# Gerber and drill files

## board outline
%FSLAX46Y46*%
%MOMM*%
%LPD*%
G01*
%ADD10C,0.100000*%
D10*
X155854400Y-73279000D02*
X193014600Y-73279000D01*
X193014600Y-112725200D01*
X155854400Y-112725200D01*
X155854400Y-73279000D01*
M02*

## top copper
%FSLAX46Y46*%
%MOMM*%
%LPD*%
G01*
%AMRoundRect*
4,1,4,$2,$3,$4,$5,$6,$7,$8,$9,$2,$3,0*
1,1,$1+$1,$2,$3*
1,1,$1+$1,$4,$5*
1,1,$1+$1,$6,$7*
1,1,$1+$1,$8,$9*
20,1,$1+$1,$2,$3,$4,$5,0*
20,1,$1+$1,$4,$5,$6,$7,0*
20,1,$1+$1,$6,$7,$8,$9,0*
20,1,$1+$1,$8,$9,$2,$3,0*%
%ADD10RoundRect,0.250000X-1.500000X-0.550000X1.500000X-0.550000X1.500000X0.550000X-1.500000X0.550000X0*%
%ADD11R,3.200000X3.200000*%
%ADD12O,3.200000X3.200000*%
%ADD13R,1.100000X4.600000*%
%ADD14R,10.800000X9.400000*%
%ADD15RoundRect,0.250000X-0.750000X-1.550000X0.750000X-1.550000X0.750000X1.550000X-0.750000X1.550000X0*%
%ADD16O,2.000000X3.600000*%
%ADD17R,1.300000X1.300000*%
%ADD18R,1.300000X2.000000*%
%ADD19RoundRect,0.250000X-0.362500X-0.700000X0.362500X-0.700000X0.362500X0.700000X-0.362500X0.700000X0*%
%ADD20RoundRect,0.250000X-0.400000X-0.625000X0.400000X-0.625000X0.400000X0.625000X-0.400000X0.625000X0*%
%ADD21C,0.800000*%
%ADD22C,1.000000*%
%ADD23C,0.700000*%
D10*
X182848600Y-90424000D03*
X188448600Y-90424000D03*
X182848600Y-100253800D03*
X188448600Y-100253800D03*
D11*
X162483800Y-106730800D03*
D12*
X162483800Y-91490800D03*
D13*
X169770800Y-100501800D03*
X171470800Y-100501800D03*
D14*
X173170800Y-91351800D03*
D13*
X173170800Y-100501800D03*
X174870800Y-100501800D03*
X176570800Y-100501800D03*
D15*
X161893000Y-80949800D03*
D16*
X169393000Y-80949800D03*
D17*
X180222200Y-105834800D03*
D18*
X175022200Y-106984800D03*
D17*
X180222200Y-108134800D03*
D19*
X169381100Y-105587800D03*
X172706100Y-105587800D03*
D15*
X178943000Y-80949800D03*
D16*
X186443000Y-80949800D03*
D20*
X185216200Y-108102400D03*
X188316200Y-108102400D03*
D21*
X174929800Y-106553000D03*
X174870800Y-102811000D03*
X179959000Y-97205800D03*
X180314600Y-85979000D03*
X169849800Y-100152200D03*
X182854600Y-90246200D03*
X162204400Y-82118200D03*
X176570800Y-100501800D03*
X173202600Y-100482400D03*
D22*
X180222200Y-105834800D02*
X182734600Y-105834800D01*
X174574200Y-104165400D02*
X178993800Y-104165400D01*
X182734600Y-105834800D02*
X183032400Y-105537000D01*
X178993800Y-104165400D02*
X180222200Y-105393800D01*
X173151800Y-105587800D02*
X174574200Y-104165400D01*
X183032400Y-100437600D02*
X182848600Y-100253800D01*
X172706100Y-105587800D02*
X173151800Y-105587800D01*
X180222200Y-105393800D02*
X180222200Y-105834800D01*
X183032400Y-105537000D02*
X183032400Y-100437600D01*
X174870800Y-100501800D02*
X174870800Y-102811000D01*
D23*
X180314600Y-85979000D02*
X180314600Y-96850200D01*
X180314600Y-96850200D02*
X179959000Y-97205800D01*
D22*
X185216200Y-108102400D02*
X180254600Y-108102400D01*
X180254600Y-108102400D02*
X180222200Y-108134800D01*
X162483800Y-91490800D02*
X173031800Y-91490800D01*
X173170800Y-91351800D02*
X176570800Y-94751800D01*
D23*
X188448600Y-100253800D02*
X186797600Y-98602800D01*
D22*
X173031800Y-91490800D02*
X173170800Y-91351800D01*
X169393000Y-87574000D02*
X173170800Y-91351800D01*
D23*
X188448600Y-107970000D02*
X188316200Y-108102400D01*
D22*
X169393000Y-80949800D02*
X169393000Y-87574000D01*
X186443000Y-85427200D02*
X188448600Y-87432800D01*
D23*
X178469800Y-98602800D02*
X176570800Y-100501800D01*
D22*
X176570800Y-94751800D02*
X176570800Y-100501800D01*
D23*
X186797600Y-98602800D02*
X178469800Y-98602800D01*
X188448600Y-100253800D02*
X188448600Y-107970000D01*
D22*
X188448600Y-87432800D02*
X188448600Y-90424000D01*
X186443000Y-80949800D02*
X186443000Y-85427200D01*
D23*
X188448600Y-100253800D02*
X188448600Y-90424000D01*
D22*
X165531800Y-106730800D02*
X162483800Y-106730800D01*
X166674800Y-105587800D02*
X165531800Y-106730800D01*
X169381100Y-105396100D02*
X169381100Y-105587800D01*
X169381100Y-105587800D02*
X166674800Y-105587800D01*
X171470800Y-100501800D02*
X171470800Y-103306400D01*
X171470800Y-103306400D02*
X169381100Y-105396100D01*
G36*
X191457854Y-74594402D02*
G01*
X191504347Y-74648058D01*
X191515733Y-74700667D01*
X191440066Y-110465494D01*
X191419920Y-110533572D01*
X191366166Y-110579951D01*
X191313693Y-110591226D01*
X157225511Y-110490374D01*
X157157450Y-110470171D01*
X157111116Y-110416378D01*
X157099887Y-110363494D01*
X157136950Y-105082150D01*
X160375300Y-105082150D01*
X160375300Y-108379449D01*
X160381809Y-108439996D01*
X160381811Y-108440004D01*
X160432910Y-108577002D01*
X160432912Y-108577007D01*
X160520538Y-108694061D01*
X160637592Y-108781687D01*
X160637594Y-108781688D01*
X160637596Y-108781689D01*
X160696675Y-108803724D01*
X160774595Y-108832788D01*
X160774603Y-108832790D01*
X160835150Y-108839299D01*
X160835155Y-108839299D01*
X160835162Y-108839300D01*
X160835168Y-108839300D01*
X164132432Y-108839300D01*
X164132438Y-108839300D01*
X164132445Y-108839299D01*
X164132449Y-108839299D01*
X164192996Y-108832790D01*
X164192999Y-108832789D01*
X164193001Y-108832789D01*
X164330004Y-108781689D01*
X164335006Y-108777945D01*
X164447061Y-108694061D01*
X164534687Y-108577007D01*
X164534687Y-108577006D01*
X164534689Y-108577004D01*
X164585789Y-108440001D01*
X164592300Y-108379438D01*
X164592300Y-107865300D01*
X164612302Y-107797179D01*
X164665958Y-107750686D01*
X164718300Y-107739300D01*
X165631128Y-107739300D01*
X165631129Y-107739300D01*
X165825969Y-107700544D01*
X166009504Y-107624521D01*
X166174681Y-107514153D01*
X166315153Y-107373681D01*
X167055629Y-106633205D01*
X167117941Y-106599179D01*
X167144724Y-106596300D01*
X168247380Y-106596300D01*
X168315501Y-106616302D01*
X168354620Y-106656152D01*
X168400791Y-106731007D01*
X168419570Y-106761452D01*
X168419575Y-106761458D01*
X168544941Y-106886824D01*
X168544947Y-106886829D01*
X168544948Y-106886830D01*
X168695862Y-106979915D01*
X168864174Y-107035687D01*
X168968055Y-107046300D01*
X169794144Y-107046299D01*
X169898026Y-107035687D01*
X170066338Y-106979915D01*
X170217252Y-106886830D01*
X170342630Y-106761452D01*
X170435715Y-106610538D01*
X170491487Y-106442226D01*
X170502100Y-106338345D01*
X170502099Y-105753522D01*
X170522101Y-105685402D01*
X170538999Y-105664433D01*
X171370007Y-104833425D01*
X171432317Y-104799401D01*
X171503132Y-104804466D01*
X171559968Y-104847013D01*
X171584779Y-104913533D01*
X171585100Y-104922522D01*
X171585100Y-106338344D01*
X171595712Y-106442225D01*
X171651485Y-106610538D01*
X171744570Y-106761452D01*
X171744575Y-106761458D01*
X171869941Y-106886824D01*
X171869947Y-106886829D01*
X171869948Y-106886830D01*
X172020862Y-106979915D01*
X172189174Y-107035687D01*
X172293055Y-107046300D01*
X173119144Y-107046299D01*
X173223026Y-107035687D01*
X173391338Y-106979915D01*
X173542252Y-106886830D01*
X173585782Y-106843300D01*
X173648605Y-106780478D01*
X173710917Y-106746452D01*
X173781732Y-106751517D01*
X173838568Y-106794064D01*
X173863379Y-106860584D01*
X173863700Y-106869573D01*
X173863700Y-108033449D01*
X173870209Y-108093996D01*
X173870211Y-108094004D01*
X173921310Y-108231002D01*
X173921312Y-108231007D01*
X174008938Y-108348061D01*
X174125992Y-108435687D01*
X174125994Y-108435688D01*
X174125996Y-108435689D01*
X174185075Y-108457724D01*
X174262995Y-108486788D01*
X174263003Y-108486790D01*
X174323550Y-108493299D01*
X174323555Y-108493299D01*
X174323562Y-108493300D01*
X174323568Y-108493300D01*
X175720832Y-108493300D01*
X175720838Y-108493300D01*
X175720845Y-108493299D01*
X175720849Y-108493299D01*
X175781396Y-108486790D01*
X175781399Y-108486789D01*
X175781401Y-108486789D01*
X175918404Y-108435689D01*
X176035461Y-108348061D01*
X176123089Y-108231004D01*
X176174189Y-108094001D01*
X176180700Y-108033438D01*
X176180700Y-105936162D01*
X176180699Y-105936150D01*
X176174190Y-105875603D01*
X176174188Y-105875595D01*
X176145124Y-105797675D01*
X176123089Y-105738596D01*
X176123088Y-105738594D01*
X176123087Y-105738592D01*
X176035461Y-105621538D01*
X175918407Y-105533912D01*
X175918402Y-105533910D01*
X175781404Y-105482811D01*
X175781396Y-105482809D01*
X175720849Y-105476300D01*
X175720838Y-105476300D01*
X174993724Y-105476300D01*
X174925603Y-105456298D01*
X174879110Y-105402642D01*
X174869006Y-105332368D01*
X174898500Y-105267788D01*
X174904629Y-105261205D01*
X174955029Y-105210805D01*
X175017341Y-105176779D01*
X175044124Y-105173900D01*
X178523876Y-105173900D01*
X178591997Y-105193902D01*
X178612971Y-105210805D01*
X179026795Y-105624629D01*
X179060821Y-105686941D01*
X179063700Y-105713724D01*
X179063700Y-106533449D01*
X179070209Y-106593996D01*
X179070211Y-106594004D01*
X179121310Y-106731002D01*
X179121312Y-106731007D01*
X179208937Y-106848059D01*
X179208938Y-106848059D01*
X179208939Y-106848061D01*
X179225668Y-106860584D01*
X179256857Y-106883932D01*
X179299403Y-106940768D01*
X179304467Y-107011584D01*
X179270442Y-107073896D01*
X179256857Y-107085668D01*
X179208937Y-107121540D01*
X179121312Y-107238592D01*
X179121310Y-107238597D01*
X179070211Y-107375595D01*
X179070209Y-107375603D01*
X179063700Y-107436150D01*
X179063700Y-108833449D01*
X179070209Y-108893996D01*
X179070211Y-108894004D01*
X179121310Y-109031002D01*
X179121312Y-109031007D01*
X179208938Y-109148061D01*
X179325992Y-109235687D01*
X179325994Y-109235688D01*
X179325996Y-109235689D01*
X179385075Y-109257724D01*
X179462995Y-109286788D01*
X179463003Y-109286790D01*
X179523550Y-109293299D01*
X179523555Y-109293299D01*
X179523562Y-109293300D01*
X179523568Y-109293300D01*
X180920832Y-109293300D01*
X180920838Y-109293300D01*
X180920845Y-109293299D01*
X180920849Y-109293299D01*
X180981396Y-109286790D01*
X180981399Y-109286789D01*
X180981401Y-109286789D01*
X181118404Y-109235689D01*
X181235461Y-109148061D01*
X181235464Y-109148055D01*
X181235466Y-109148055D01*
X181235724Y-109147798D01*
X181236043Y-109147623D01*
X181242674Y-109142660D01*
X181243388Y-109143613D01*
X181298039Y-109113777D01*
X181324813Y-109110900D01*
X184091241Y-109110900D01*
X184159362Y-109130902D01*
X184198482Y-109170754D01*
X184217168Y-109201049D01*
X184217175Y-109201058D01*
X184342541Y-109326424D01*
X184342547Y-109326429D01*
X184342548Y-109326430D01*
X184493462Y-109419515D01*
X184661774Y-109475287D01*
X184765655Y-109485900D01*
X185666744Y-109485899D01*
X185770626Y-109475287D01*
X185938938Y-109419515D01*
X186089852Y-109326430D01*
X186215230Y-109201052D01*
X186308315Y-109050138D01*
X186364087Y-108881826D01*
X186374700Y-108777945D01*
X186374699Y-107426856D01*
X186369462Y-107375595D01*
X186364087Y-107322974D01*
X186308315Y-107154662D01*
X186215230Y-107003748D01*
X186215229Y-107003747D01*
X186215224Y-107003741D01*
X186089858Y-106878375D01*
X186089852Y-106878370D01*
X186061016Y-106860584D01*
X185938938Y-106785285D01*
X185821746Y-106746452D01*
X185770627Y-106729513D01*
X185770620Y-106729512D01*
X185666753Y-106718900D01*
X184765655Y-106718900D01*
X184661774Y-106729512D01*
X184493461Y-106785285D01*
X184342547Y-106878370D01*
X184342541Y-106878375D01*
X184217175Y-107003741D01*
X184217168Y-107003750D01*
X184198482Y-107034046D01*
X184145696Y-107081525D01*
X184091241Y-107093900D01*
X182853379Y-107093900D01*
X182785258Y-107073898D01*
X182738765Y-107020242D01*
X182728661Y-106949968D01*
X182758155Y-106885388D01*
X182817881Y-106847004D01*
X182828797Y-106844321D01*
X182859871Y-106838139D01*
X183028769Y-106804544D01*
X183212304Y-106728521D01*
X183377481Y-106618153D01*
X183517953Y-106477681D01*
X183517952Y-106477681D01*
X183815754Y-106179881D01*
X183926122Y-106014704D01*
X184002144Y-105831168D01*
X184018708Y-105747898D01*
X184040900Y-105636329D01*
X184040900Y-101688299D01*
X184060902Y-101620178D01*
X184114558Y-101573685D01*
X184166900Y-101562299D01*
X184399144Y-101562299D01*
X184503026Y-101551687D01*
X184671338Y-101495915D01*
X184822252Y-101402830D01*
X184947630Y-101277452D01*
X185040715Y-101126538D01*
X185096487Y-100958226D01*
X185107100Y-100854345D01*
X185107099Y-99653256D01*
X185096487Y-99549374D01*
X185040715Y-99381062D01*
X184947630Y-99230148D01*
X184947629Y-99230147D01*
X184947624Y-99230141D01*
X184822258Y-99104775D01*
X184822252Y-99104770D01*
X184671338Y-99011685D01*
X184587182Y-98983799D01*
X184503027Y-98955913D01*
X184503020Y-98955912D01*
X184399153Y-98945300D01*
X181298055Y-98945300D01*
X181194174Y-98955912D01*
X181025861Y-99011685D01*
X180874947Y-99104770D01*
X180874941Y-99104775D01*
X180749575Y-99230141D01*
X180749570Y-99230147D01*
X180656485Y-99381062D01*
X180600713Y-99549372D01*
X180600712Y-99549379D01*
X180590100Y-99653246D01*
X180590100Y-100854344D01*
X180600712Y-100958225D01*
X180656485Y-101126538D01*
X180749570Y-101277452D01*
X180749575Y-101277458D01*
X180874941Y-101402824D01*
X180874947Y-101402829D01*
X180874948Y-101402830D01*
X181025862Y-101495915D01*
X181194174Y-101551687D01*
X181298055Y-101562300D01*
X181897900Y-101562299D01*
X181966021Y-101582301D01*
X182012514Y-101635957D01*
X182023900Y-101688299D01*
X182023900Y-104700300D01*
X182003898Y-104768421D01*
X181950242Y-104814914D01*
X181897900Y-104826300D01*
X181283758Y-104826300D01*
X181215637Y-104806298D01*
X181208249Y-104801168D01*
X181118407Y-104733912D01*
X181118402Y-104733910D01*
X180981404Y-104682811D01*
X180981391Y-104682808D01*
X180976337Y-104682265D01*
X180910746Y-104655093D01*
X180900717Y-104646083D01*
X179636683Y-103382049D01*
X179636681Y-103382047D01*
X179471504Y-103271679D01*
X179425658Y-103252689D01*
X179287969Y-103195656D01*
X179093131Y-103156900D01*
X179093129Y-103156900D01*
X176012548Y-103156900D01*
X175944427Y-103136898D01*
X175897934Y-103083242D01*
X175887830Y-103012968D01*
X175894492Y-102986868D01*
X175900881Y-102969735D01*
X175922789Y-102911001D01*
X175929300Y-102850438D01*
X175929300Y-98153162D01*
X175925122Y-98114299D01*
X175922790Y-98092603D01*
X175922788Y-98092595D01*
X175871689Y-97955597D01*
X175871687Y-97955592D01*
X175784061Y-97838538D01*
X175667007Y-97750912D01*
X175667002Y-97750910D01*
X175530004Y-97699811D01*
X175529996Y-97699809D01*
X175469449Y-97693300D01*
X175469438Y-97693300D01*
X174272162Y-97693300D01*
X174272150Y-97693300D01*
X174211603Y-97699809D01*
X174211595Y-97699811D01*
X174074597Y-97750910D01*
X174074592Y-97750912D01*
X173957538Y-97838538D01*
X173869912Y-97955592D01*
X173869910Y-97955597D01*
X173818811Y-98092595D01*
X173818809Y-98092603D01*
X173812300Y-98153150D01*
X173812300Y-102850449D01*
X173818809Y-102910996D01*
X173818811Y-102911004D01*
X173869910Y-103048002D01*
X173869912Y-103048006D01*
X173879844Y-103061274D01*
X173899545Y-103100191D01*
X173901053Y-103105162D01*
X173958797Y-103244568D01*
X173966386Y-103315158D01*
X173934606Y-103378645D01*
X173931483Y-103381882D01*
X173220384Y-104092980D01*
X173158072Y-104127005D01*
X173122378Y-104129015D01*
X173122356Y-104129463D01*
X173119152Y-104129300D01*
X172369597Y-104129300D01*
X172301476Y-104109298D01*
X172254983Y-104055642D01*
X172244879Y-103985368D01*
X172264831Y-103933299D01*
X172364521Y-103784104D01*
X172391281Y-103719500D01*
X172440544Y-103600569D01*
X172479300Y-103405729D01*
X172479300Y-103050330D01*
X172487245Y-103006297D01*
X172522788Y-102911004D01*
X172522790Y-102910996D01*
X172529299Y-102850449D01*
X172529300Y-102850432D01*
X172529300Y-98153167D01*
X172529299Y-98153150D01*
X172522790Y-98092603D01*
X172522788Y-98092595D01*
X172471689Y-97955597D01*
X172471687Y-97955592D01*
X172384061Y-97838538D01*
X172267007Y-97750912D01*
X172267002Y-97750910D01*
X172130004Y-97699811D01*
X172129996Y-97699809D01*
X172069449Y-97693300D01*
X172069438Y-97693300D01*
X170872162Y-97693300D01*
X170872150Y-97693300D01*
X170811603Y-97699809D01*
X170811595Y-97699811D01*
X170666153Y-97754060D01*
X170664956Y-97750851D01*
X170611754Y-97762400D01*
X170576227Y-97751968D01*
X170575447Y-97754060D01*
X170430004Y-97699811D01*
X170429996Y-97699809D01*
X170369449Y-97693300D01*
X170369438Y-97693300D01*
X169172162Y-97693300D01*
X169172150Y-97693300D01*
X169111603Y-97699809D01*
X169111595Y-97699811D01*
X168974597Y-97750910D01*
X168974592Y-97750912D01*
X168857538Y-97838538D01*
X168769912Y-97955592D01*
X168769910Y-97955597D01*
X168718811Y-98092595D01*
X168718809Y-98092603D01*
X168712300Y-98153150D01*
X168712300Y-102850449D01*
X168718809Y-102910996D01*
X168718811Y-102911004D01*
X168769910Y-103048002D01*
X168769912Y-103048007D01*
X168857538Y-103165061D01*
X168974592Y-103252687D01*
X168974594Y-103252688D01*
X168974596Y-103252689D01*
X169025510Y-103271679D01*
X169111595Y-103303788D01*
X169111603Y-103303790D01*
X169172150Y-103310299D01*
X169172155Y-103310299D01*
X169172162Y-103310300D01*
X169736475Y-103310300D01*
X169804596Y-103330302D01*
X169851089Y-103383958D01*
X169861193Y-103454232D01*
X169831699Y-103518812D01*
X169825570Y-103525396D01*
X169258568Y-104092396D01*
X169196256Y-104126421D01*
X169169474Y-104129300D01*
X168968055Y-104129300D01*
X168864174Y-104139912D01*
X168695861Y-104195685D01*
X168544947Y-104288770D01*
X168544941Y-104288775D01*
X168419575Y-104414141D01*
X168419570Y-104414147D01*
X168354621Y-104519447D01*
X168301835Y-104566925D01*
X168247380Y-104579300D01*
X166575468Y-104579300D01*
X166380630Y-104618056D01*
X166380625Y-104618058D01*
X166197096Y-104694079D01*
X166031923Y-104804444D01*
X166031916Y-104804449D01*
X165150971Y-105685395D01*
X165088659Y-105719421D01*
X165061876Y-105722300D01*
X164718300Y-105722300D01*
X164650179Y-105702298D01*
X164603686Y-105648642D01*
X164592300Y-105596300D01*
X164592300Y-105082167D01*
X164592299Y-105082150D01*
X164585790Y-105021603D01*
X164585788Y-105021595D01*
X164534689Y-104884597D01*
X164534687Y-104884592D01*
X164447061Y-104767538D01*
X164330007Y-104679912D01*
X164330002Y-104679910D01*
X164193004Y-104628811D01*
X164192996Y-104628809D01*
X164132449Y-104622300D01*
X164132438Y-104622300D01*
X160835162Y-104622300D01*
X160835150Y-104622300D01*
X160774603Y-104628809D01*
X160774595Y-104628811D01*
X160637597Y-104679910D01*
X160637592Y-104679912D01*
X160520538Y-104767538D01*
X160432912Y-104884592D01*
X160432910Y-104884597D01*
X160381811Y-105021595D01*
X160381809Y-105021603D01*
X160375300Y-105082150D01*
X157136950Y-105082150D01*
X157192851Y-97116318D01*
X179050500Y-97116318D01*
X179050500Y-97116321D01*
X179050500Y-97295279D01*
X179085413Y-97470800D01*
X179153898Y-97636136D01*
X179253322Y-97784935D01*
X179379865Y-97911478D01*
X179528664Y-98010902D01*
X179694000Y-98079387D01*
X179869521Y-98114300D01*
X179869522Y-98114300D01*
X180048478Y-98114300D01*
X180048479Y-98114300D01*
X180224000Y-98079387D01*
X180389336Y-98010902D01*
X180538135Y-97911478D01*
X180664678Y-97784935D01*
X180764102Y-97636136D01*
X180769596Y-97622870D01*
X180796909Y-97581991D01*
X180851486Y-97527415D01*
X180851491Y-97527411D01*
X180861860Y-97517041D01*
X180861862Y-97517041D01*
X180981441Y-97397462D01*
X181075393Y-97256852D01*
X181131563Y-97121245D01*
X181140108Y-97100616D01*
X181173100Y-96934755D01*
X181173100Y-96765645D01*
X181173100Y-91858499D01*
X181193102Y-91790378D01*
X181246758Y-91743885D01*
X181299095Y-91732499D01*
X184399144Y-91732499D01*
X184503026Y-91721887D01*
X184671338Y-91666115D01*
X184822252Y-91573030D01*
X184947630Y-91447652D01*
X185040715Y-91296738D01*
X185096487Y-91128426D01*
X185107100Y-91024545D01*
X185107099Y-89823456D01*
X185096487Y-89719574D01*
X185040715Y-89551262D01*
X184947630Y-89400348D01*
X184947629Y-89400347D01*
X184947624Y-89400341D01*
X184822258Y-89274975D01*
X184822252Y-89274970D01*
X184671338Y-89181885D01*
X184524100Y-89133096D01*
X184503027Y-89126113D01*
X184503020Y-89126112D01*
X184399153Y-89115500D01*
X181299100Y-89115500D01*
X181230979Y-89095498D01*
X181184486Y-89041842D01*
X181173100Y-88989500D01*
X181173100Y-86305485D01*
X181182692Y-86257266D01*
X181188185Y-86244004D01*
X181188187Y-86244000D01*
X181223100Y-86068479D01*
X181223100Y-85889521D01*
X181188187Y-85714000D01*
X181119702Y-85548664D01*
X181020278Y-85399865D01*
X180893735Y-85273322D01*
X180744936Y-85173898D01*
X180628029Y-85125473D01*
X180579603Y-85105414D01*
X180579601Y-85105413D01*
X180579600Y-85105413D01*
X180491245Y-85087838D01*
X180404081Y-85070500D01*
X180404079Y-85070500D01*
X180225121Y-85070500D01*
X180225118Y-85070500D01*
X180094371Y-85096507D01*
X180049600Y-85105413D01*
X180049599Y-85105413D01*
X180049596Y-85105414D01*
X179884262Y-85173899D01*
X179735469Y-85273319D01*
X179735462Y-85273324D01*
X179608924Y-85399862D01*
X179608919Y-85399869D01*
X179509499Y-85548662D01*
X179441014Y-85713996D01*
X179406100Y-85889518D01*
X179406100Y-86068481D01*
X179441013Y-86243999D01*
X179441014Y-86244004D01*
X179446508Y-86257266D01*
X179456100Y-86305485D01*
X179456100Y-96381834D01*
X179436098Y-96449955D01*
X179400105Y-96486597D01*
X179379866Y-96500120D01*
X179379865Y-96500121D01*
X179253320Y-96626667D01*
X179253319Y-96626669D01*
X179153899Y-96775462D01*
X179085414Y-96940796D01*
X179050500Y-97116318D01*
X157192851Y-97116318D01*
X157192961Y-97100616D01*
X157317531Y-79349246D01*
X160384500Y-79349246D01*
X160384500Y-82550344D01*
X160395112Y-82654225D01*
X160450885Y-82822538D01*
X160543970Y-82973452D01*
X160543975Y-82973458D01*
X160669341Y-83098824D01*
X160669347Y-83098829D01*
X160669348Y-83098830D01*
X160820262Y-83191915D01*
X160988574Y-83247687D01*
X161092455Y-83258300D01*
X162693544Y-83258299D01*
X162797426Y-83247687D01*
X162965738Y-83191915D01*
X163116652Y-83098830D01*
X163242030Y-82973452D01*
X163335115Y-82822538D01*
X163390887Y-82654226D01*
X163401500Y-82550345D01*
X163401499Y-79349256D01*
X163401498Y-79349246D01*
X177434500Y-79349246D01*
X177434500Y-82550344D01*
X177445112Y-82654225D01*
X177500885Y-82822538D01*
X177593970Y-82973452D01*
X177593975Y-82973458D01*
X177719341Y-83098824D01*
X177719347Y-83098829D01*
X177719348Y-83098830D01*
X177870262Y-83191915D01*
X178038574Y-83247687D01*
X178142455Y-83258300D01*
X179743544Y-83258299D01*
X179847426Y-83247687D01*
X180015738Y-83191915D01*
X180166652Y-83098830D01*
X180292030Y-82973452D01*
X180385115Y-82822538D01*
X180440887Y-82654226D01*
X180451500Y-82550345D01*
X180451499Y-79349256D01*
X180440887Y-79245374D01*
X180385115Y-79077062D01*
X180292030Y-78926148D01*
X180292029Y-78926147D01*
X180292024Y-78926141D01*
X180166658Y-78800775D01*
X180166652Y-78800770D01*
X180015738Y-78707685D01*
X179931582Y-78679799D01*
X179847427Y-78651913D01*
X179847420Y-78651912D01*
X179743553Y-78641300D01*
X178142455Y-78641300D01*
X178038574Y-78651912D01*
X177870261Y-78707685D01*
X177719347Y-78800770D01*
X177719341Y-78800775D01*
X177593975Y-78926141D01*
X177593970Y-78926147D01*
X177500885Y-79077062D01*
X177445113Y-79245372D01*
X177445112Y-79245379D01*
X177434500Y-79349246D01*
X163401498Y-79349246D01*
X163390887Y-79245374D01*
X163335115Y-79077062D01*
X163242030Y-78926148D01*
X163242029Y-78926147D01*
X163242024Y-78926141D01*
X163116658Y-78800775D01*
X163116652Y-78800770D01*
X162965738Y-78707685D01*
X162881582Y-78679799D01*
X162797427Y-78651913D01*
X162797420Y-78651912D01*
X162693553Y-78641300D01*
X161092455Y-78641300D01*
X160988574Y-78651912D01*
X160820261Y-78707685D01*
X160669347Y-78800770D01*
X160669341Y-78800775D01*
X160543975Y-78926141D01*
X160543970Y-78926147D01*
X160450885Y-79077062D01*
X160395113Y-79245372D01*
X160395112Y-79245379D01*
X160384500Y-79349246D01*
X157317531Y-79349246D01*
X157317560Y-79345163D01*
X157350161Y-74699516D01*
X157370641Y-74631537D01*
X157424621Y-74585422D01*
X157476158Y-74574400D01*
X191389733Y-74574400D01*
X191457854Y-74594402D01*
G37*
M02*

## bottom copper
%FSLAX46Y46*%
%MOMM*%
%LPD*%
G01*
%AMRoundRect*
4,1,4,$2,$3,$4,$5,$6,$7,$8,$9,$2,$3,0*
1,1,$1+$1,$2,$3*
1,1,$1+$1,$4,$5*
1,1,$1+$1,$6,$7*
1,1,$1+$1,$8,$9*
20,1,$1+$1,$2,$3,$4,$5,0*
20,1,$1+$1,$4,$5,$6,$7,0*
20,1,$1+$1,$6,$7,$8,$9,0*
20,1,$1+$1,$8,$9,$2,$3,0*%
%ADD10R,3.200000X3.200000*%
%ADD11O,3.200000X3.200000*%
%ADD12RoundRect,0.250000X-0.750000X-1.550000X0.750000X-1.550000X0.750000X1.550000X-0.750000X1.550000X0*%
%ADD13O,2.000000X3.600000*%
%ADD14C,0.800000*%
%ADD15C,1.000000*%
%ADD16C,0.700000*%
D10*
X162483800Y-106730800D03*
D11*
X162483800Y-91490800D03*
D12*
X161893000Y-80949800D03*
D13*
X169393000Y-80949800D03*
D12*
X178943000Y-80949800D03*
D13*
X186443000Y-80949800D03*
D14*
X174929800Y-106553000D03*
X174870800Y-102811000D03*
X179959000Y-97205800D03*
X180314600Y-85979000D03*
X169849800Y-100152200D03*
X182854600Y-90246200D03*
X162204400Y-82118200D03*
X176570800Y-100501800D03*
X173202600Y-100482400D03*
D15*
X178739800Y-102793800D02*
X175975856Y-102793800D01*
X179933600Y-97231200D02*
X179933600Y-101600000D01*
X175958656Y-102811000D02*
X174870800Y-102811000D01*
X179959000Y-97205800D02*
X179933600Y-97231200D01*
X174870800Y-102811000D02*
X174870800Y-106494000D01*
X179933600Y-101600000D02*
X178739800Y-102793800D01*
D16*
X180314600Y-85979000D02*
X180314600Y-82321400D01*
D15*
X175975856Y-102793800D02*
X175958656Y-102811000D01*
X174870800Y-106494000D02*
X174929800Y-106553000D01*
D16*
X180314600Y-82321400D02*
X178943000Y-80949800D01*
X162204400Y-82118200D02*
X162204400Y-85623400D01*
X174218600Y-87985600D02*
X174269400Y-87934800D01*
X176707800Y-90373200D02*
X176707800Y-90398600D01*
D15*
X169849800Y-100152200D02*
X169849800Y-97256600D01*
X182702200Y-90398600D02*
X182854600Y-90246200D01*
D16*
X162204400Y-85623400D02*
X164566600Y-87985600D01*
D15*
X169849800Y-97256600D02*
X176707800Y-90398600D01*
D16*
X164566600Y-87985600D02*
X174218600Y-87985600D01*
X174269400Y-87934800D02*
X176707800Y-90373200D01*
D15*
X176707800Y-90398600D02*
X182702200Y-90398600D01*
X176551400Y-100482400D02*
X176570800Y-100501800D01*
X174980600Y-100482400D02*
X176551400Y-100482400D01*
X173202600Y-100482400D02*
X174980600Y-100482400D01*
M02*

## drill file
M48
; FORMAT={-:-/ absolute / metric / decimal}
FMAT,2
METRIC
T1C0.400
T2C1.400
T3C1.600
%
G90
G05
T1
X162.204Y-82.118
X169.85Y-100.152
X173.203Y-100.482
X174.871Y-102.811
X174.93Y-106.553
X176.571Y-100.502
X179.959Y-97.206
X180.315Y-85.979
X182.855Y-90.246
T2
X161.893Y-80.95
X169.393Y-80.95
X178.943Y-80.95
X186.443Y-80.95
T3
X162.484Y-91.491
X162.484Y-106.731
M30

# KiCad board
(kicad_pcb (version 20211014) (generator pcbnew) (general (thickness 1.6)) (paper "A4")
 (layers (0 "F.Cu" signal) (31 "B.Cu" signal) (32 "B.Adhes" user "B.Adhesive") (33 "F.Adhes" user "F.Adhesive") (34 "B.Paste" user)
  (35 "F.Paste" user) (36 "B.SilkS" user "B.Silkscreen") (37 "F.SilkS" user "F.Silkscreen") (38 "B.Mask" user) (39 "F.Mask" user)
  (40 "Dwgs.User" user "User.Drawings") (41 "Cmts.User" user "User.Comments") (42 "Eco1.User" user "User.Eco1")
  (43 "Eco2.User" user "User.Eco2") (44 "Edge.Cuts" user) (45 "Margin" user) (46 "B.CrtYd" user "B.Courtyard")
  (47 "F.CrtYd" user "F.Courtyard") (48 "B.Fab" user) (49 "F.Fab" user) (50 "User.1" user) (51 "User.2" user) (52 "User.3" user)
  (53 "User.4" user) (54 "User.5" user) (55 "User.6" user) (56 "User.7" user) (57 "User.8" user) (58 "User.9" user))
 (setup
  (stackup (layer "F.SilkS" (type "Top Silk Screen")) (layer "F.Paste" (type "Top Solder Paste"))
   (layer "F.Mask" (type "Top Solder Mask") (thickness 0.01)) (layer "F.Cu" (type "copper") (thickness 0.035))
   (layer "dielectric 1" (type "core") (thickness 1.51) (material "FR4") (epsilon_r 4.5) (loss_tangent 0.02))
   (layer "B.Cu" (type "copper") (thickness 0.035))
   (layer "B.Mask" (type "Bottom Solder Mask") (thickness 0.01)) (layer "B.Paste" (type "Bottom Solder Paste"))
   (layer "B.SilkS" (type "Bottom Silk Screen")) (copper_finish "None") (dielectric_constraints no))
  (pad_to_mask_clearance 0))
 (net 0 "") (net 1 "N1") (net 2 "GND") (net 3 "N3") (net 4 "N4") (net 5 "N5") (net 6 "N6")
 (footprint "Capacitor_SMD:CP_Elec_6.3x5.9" (layer "F.Cu") (at 185.6486 90.424)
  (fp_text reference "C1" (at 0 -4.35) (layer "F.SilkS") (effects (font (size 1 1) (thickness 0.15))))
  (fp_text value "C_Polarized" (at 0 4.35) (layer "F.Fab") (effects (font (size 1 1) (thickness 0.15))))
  (pad "1" smd roundrect (at -2.8 0) (size 3.5 1.6) (layers "F.Cu" "F.Paste" "F.Mask") (roundrect_rratio 0.15625) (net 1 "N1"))
  (pad "2" smd roundrect (at 2.8 0) (size 3.5 1.6) (layers "F.Cu" "F.Paste" "F.Mask") (roundrect_rratio 0.15625) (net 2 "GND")))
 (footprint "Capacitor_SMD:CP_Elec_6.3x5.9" (layer "F.Cu") (at 185.6486 100.2538)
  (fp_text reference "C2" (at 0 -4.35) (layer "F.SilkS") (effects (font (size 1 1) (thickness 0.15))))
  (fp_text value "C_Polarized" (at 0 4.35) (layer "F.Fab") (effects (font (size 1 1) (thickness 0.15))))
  (pad "1" smd roundrect (at -2.8 0) (size 3.5 1.6) (layers "F.Cu" "F.Paste" "F.Mask") (roundrect_rratio 0.15625) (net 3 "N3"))
  (pad "2" smd roundrect (at 2.8 0) (size 3.5 1.6) (layers "F.Cu" "F.Paste" "F.Mask") (roundrect_rratio 0.15625) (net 2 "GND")))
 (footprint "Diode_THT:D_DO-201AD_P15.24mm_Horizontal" (layer "F.Cu") (at 162.4838 106.7308 90)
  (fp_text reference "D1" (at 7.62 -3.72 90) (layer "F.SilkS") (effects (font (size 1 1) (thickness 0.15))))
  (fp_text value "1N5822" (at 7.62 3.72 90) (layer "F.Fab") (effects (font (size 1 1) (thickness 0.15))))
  (pad "1" thru_hole rect (at 0 0 90) (size 3.2 3.2) (drill 1.6) (layers *.Cu *.Mask) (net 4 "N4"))
  (pad "2" thru_hole oval (at 15.24 0 90) (size 3.2 3.2) (drill 1.6) (layers *.Cu *.Mask) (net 2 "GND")))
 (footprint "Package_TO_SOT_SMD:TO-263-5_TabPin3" (layer "F.Cu") (at 173.1708 94.7268 90)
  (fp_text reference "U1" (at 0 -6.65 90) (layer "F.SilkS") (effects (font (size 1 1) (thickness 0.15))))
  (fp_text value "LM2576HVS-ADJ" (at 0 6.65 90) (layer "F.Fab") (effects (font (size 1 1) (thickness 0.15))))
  (pad "" smd rect (at 5.8 2.775 90) (size 4.55 5.25) (layers "F.Paste"))
  (pad "" smd rect (at 0.95 2.775 90) (size 4.55 5.25) (layers "F.Paste"))
  (pad "" smd rect (at 0.95 -2.775 90) (size 4.55 5.25) (layers "F.Paste"))
  (pad "" smd rect (at 5.8 -2.775 90) (size 4.55 5.25) (layers "F.Paste"))
  (pad "1" smd rect (at -5.775 -3.4 90) (size 4.6 1.1) (layers "F.Cu" "F.Paste" "F.Mask") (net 1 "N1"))
  (pad "2" smd rect (at -5.775 -1.7 90) (size 4.6 1.1) (layers "F.Cu" "F.Paste" "F.Mask") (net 4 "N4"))
  (pad "3" smd rect (at 3.375 0 90) (size 9.4 10.8) (layers "F.Cu" "F.Mask") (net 2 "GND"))
  (pad "3" smd rect (at -5.775 0 90) (size 4.6 1.1) (layers "F.Cu" "F.Paste" "F.Mask") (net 2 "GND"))
  (pad "4" smd rect (at -5.775 1.7 90) (size 4.6 1.1) (layers "F.Cu" "F.Paste" "F.Mask") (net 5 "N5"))
  (pad "5" smd rect (at -5.775 3.4 90) (size 4.6 1.1) (layers "F.Cu" "F.Paste" "F.Mask") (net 2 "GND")))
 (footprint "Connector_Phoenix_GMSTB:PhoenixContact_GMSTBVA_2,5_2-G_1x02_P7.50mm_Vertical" (layer "F.Cu") (at 161.893 80.9498)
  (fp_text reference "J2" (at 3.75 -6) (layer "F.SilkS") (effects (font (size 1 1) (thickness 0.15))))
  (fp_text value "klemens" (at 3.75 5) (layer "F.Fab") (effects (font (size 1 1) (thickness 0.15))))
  (pad "1" thru_hole roundrect (at 0 0) (size 2 3.6) (drill 1.4) (layers *.Cu *.Mask) (roundrect_rratio 0.125) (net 1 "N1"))
  (pad "2" thru_hole oval (at 7.5 0) (size 2 3.6) (drill 1.4) (layers *.Cu *.Mask) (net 2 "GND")))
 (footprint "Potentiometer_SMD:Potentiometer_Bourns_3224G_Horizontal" (layer "F.Cu") (at 177.6222 106.9848)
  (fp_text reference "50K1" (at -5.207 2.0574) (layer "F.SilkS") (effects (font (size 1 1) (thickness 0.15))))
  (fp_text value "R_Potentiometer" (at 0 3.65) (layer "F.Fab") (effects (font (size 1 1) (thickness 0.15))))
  (pad "1" smd rect (at 2.6 -1.15) (size 1.3 1.3) (layers "F.Cu" "F.Paste" "F.Mask") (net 3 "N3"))
  (pad "2" smd rect (at -2.6 0) (size 1.3 2) (layers "F.Cu" "F.Paste" "F.Mask") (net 5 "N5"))
  (pad "3" smd rect (at 2.6 1.15) (size 1.3 1.3) (layers "F.Cu" "F.Paste" "F.Mask") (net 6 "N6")))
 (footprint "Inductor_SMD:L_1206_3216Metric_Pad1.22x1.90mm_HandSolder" (layer "F.Cu") (at 171.0436 105.5878)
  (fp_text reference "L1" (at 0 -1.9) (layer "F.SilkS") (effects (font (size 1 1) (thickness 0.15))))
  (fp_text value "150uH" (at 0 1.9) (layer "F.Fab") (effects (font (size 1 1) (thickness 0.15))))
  (pad "1" smd roundrect (at -1.6625 0) (size 1.225 1.9) (layers "F.Cu" "F.Paste" "F.Mask") (roundrect_rratio 0.2040816327) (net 4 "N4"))
  (pad "2" smd roundrect (at 1.6625 0) (size 1.225 1.9) (layers "F.Cu" "F.Paste" "F.Mask") (roundrect_rratio 0.2040816327) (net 3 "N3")))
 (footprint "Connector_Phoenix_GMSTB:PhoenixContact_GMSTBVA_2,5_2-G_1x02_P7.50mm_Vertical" (layer "F.Cu") (at 178.943 80.9498)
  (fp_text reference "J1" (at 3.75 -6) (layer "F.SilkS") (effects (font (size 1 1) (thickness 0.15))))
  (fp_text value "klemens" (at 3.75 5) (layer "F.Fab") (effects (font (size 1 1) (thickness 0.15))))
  (pad "1" thru_hole roundrect (at 0 0) (size 2 3.6) (drill 1.4) (layers *.Cu *.Mask) (roundrect_rratio 0.125) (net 5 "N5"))
  (pad "2" thru_hole oval (at 7.5 0) (size 2 3.6) (drill 1.4) (layers *.Cu *.Mask) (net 2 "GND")))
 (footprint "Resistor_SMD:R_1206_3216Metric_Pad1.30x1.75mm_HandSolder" (layer "F.Cu") (at 186.7662 108.1024)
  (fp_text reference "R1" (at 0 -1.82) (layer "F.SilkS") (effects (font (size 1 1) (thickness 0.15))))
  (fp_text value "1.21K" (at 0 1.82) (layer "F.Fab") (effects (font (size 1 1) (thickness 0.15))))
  (pad "1" smd roundrect (at -1.55 0) (size 1.3 1.75) (layers "F.Cu" "F.Paste" "F.Mask") (roundrect_rratio 0.1923076923) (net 6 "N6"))
  (pad "2" smd roundrect (at 1.55 0) (size 1.3 1.75) (layers "F.Cu" "F.Paste" "F.Mask") (roundrect_rratio 0.1923076923) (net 2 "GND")))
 (gr_rect (start 155.8544 73.279) (end 193.0146 112.7252) (layer "Edge.Cuts") (width 0.1) (fill none))
 (segment (start 180.2222 105.8348) (end 182.7346 105.8348) (width 1) (layer "F.Cu") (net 3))
 (segment (start 174.5742 104.1654) (end 178.9938 104.1654) (width 1) (layer "F.Cu") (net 3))
 (segment (start 182.7346 105.8348) (end 183.0324 105.537) (width 1) (layer "F.Cu") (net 3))
 (segment (start 178.9938 104.1654) (end 180.2222 105.3938) (width 1) (layer "F.Cu") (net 3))
 (segment (start 173.1518 105.5878) (end 174.5742 104.1654) (width 1) (layer "F.Cu") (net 3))
 (segment (start 183.0324 100.4376) (end 182.8486 100.2538) (width 1) (layer "F.Cu") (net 3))
 (segment (start 172.7061 105.5878) (end 173.1518 105.5878) (width 1) (layer "F.Cu") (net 3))
 (segment (start 180.2222 105.3938) (end 180.2222 105.8348) (width 1) (layer "F.Cu") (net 3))
 (segment (start 183.0324 105.537) (end 183.0324 100.4376) (width 1) (layer "F.Cu") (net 3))
 (segment (start 174.8708 100.5018) (end 174.8708 102.811) (width 1) (layer "F.Cu") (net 5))
 (segment (start 180.3146 85.979) (end 180.3146 96.8502) (width 0.7) (layer "F.Cu") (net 5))
 (segment (start 180.3146 96.8502) (end 179.959 97.2058) (width 0.7) (layer "F.Cu") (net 5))
 (via (at 174.9298 106.553) (size 0.8) (drill 0.4) (layers "F.Cu" "B.Cu") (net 5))
 (via (at 174.8708 102.811) (size 0.8) (drill 0.4) (layers "F.Cu" "B.Cu") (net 5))
 (via (at 179.959 97.2058) (size 0.8) (drill 0.4) (layers "F.Cu" "B.Cu") (free) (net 5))
 (via (at 180.3146 85.979) (size 0.8) (drill 0.4) (layers "F.Cu" "B.Cu") (free) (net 5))
 (segment (start 178.7398 102.7938) (end 175.975856 102.7938) (width 1) (layer "B.Cu") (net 5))
 (segment (start 179.9336 97.2312) (end 179.9336 101.6) (width 1) (layer "B.Cu") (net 5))
 (segment (start 175.958656 102.811) (end 174.8708 102.811) (width 1) (layer "B.Cu") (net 5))
 (segment (start 179.959 97.2058) (end 179.9336 97.2312) (width 1) (layer "B.Cu") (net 5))
 (segment (start 174.8708 102.811) (end 174.8708 106.494) (width 1) (layer "B.Cu") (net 5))
 (segment (start 179.9336 101.6) (end 178.7398 102.7938) (width 1) (layer "B.Cu") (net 5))
 (segment (start 180.3146 85.979) (end 180.3146 82.3214) (width 0.7) (layer "B.Cu") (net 5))
 (segment (start 175.975856 102.7938) (end 175.958656 102.811) (width 1) (layer "B.Cu") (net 5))
 (segment (start 174.8708 106.494) (end 174.9298 106.553) (width 1) (layer "B.Cu") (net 5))
 (segment (start 180.3146 82.3214) (end 178.943 80.9498) (width 0.7) (layer "B.Cu") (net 5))
 (segment (start 185.2162 108.1024) (end 180.2546 108.1024) (width 1) (layer "F.Cu") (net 6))
 (segment (start 180.2546 108.1024) (end 180.2222 108.1348) (width 1) (layer "F.Cu") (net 6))
 (via (at 169.8498 100.1522) (size 0.8) (drill 0.4) (layers "F.Cu" "B.Cu") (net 1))
 (via (at 182.8546 90.2462) (size 0.8) (drill 0.4) (layers "F.Cu" "B.Cu") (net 1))
 (via (at 162.2044 82.1182) (size 0.8) (drill 0.4) (layers "F.Cu" "B.Cu") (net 1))
 (segment (start 162.2044 82.1182) (end 162.2044 85.6234) (width 0.7) (layer "B.Cu") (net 1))
 (segment (start 174.2186 87.9856) (end 174.2694 87.9348) (width 0.7) (layer "B.Cu") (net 1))
 (segment (start 176.7078 90.3732) (end 176.7078 90.3986) (width 0.7) (layer "B.Cu") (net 1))
 (segment (start 169.8498 100.1522) (end 169.8498 97.2566) (width 1) (layer "B.Cu") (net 1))
 (segment (start 182.7022 90.3986) (end 182.8546 90.2462) (width 1) (layer "B.Cu") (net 1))
 (segment (start 162.2044 85.6234) (end 164.5666 87.9856) (width 0.7) (layer "B.Cu") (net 1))
 (segment (start 169.8498 97.2566) (end 176.7078 90.3986) (width 1) (layer "B.Cu") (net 1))
 (segment (start 164.5666 87.9856) (end 174.2186 87.9856) (width 0.7) (layer "B.Cu") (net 1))
 (segment (start 174.2694 87.9348) (end 176.7078 90.3732) (width 0.7) (layer "B.Cu") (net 1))
 (segment (start 176.7078 90.3986) (end 182.7022 90.3986) (width 1) (layer "B.Cu") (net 1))
 (segment (start 162.4838 91.4908) (end 173.0318 91.4908) (width 1) (layer "F.Cu") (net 2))
 (segment (start 173.1708 91.3518) (end 176.5708 94.7518) (width 1) (layer "F.Cu") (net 2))
 (segment (start 188.4486 100.2538) (end 186.7976 98.6028) (width 0.7) (layer "F.Cu") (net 2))
 (segment (start 173.0318 91.4908) (end 173.1708 91.3518) (width 1) (layer "F.Cu") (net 2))
 (segment (start 169.393 87.574) (end 173.1708 91.3518) (width 1) (layer "F.Cu") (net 2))
 (segment (start 188.4486 107.97) (end 188.3162 108.1024) (width 0.7) (layer "F.Cu") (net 2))
 (segment (start 169.393 80.9498) (end 169.393 87.574) (width 1) (layer "F.Cu") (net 2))
 (segment (start 186.443 85.4272) (end 188.4486 87.4328) (width 1) (layer "F.Cu") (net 2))
 (segment (start 178.4698 98.6028) (end 176.5708 100.5018) (width 0.7) (layer "F.Cu") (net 2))
 (segment (start 176.5708 94.7518) (end 176.5708 100.5018) (width 1) (layer "F.Cu") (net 2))
 (segment (start 186.7976 98.6028) (end 178.4698 98.6028) (width 0.7) (layer "F.Cu") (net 2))
 (segment (start 188.4486 100.2538) (end 188.4486 107.97) (width 0.7) (layer "F.Cu") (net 2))
 (segment (start 188.4486 87.4328) (end 188.4486 90.424) (width 1) (layer "F.Cu") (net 2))
 (segment (start 186.443 80.9498) (end 186.443 85.4272) (width 1) (layer "F.Cu") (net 2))
 (segment (start 188.4486 100.2538) (end 188.4486 90.424) (width 0.7) (layer "F.Cu") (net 2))
 (via (at 176.5708 100.5018) (size 0.8) (drill 0.4) (layers "F.Cu" "B.Cu") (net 2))
 (via (at 173.2026 100.4824) (size 0.8) (drill 0.4) (layers "F.Cu" "B.Cu") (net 2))
 (segment (start 176.5514 100.4824) (end 176.5708 100.5018) (width 1) (layer "B.Cu") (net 2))
 (segment (start 174.9806 100.4824) (end 176.5514 100.4824) (width 1) (layer "B.Cu") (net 2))
 (segment (start 173.2026 100.4824) (end 174.9806 100.4824) (width 1) (layer "B.Cu") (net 2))
 (segment (start 165.5318 106.7308) (end 162.4838 106.7308) (width 1) (layer "F.Cu") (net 4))
 (segment (start 166.6748 105.5878) (end 165.5318 106.7308) (width 1) (layer "F.Cu") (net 4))
 (segment (start 169.3811 105.3961) (end 169.3811 105.5878) (width 1) (layer "F.Cu") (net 4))
 (segment (start 169.3811 105.5878) (end 166.6748 105.5878) (width 1) (layer "F.Cu") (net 4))
 (segment (start 171.4708 100.5018) (end 171.4708 103.3064) (width 1) (layer "F.Cu") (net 4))
 (segment (start 171.4708 103.3064) (end 169.3811 105.3961) (width 1) (layer "F.Cu") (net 4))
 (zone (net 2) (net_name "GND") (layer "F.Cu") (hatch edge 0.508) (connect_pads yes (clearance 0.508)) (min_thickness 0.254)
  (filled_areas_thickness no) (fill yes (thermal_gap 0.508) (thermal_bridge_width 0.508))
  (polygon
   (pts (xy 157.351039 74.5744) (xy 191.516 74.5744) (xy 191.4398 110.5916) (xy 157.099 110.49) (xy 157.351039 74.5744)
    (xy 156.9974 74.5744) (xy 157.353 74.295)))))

